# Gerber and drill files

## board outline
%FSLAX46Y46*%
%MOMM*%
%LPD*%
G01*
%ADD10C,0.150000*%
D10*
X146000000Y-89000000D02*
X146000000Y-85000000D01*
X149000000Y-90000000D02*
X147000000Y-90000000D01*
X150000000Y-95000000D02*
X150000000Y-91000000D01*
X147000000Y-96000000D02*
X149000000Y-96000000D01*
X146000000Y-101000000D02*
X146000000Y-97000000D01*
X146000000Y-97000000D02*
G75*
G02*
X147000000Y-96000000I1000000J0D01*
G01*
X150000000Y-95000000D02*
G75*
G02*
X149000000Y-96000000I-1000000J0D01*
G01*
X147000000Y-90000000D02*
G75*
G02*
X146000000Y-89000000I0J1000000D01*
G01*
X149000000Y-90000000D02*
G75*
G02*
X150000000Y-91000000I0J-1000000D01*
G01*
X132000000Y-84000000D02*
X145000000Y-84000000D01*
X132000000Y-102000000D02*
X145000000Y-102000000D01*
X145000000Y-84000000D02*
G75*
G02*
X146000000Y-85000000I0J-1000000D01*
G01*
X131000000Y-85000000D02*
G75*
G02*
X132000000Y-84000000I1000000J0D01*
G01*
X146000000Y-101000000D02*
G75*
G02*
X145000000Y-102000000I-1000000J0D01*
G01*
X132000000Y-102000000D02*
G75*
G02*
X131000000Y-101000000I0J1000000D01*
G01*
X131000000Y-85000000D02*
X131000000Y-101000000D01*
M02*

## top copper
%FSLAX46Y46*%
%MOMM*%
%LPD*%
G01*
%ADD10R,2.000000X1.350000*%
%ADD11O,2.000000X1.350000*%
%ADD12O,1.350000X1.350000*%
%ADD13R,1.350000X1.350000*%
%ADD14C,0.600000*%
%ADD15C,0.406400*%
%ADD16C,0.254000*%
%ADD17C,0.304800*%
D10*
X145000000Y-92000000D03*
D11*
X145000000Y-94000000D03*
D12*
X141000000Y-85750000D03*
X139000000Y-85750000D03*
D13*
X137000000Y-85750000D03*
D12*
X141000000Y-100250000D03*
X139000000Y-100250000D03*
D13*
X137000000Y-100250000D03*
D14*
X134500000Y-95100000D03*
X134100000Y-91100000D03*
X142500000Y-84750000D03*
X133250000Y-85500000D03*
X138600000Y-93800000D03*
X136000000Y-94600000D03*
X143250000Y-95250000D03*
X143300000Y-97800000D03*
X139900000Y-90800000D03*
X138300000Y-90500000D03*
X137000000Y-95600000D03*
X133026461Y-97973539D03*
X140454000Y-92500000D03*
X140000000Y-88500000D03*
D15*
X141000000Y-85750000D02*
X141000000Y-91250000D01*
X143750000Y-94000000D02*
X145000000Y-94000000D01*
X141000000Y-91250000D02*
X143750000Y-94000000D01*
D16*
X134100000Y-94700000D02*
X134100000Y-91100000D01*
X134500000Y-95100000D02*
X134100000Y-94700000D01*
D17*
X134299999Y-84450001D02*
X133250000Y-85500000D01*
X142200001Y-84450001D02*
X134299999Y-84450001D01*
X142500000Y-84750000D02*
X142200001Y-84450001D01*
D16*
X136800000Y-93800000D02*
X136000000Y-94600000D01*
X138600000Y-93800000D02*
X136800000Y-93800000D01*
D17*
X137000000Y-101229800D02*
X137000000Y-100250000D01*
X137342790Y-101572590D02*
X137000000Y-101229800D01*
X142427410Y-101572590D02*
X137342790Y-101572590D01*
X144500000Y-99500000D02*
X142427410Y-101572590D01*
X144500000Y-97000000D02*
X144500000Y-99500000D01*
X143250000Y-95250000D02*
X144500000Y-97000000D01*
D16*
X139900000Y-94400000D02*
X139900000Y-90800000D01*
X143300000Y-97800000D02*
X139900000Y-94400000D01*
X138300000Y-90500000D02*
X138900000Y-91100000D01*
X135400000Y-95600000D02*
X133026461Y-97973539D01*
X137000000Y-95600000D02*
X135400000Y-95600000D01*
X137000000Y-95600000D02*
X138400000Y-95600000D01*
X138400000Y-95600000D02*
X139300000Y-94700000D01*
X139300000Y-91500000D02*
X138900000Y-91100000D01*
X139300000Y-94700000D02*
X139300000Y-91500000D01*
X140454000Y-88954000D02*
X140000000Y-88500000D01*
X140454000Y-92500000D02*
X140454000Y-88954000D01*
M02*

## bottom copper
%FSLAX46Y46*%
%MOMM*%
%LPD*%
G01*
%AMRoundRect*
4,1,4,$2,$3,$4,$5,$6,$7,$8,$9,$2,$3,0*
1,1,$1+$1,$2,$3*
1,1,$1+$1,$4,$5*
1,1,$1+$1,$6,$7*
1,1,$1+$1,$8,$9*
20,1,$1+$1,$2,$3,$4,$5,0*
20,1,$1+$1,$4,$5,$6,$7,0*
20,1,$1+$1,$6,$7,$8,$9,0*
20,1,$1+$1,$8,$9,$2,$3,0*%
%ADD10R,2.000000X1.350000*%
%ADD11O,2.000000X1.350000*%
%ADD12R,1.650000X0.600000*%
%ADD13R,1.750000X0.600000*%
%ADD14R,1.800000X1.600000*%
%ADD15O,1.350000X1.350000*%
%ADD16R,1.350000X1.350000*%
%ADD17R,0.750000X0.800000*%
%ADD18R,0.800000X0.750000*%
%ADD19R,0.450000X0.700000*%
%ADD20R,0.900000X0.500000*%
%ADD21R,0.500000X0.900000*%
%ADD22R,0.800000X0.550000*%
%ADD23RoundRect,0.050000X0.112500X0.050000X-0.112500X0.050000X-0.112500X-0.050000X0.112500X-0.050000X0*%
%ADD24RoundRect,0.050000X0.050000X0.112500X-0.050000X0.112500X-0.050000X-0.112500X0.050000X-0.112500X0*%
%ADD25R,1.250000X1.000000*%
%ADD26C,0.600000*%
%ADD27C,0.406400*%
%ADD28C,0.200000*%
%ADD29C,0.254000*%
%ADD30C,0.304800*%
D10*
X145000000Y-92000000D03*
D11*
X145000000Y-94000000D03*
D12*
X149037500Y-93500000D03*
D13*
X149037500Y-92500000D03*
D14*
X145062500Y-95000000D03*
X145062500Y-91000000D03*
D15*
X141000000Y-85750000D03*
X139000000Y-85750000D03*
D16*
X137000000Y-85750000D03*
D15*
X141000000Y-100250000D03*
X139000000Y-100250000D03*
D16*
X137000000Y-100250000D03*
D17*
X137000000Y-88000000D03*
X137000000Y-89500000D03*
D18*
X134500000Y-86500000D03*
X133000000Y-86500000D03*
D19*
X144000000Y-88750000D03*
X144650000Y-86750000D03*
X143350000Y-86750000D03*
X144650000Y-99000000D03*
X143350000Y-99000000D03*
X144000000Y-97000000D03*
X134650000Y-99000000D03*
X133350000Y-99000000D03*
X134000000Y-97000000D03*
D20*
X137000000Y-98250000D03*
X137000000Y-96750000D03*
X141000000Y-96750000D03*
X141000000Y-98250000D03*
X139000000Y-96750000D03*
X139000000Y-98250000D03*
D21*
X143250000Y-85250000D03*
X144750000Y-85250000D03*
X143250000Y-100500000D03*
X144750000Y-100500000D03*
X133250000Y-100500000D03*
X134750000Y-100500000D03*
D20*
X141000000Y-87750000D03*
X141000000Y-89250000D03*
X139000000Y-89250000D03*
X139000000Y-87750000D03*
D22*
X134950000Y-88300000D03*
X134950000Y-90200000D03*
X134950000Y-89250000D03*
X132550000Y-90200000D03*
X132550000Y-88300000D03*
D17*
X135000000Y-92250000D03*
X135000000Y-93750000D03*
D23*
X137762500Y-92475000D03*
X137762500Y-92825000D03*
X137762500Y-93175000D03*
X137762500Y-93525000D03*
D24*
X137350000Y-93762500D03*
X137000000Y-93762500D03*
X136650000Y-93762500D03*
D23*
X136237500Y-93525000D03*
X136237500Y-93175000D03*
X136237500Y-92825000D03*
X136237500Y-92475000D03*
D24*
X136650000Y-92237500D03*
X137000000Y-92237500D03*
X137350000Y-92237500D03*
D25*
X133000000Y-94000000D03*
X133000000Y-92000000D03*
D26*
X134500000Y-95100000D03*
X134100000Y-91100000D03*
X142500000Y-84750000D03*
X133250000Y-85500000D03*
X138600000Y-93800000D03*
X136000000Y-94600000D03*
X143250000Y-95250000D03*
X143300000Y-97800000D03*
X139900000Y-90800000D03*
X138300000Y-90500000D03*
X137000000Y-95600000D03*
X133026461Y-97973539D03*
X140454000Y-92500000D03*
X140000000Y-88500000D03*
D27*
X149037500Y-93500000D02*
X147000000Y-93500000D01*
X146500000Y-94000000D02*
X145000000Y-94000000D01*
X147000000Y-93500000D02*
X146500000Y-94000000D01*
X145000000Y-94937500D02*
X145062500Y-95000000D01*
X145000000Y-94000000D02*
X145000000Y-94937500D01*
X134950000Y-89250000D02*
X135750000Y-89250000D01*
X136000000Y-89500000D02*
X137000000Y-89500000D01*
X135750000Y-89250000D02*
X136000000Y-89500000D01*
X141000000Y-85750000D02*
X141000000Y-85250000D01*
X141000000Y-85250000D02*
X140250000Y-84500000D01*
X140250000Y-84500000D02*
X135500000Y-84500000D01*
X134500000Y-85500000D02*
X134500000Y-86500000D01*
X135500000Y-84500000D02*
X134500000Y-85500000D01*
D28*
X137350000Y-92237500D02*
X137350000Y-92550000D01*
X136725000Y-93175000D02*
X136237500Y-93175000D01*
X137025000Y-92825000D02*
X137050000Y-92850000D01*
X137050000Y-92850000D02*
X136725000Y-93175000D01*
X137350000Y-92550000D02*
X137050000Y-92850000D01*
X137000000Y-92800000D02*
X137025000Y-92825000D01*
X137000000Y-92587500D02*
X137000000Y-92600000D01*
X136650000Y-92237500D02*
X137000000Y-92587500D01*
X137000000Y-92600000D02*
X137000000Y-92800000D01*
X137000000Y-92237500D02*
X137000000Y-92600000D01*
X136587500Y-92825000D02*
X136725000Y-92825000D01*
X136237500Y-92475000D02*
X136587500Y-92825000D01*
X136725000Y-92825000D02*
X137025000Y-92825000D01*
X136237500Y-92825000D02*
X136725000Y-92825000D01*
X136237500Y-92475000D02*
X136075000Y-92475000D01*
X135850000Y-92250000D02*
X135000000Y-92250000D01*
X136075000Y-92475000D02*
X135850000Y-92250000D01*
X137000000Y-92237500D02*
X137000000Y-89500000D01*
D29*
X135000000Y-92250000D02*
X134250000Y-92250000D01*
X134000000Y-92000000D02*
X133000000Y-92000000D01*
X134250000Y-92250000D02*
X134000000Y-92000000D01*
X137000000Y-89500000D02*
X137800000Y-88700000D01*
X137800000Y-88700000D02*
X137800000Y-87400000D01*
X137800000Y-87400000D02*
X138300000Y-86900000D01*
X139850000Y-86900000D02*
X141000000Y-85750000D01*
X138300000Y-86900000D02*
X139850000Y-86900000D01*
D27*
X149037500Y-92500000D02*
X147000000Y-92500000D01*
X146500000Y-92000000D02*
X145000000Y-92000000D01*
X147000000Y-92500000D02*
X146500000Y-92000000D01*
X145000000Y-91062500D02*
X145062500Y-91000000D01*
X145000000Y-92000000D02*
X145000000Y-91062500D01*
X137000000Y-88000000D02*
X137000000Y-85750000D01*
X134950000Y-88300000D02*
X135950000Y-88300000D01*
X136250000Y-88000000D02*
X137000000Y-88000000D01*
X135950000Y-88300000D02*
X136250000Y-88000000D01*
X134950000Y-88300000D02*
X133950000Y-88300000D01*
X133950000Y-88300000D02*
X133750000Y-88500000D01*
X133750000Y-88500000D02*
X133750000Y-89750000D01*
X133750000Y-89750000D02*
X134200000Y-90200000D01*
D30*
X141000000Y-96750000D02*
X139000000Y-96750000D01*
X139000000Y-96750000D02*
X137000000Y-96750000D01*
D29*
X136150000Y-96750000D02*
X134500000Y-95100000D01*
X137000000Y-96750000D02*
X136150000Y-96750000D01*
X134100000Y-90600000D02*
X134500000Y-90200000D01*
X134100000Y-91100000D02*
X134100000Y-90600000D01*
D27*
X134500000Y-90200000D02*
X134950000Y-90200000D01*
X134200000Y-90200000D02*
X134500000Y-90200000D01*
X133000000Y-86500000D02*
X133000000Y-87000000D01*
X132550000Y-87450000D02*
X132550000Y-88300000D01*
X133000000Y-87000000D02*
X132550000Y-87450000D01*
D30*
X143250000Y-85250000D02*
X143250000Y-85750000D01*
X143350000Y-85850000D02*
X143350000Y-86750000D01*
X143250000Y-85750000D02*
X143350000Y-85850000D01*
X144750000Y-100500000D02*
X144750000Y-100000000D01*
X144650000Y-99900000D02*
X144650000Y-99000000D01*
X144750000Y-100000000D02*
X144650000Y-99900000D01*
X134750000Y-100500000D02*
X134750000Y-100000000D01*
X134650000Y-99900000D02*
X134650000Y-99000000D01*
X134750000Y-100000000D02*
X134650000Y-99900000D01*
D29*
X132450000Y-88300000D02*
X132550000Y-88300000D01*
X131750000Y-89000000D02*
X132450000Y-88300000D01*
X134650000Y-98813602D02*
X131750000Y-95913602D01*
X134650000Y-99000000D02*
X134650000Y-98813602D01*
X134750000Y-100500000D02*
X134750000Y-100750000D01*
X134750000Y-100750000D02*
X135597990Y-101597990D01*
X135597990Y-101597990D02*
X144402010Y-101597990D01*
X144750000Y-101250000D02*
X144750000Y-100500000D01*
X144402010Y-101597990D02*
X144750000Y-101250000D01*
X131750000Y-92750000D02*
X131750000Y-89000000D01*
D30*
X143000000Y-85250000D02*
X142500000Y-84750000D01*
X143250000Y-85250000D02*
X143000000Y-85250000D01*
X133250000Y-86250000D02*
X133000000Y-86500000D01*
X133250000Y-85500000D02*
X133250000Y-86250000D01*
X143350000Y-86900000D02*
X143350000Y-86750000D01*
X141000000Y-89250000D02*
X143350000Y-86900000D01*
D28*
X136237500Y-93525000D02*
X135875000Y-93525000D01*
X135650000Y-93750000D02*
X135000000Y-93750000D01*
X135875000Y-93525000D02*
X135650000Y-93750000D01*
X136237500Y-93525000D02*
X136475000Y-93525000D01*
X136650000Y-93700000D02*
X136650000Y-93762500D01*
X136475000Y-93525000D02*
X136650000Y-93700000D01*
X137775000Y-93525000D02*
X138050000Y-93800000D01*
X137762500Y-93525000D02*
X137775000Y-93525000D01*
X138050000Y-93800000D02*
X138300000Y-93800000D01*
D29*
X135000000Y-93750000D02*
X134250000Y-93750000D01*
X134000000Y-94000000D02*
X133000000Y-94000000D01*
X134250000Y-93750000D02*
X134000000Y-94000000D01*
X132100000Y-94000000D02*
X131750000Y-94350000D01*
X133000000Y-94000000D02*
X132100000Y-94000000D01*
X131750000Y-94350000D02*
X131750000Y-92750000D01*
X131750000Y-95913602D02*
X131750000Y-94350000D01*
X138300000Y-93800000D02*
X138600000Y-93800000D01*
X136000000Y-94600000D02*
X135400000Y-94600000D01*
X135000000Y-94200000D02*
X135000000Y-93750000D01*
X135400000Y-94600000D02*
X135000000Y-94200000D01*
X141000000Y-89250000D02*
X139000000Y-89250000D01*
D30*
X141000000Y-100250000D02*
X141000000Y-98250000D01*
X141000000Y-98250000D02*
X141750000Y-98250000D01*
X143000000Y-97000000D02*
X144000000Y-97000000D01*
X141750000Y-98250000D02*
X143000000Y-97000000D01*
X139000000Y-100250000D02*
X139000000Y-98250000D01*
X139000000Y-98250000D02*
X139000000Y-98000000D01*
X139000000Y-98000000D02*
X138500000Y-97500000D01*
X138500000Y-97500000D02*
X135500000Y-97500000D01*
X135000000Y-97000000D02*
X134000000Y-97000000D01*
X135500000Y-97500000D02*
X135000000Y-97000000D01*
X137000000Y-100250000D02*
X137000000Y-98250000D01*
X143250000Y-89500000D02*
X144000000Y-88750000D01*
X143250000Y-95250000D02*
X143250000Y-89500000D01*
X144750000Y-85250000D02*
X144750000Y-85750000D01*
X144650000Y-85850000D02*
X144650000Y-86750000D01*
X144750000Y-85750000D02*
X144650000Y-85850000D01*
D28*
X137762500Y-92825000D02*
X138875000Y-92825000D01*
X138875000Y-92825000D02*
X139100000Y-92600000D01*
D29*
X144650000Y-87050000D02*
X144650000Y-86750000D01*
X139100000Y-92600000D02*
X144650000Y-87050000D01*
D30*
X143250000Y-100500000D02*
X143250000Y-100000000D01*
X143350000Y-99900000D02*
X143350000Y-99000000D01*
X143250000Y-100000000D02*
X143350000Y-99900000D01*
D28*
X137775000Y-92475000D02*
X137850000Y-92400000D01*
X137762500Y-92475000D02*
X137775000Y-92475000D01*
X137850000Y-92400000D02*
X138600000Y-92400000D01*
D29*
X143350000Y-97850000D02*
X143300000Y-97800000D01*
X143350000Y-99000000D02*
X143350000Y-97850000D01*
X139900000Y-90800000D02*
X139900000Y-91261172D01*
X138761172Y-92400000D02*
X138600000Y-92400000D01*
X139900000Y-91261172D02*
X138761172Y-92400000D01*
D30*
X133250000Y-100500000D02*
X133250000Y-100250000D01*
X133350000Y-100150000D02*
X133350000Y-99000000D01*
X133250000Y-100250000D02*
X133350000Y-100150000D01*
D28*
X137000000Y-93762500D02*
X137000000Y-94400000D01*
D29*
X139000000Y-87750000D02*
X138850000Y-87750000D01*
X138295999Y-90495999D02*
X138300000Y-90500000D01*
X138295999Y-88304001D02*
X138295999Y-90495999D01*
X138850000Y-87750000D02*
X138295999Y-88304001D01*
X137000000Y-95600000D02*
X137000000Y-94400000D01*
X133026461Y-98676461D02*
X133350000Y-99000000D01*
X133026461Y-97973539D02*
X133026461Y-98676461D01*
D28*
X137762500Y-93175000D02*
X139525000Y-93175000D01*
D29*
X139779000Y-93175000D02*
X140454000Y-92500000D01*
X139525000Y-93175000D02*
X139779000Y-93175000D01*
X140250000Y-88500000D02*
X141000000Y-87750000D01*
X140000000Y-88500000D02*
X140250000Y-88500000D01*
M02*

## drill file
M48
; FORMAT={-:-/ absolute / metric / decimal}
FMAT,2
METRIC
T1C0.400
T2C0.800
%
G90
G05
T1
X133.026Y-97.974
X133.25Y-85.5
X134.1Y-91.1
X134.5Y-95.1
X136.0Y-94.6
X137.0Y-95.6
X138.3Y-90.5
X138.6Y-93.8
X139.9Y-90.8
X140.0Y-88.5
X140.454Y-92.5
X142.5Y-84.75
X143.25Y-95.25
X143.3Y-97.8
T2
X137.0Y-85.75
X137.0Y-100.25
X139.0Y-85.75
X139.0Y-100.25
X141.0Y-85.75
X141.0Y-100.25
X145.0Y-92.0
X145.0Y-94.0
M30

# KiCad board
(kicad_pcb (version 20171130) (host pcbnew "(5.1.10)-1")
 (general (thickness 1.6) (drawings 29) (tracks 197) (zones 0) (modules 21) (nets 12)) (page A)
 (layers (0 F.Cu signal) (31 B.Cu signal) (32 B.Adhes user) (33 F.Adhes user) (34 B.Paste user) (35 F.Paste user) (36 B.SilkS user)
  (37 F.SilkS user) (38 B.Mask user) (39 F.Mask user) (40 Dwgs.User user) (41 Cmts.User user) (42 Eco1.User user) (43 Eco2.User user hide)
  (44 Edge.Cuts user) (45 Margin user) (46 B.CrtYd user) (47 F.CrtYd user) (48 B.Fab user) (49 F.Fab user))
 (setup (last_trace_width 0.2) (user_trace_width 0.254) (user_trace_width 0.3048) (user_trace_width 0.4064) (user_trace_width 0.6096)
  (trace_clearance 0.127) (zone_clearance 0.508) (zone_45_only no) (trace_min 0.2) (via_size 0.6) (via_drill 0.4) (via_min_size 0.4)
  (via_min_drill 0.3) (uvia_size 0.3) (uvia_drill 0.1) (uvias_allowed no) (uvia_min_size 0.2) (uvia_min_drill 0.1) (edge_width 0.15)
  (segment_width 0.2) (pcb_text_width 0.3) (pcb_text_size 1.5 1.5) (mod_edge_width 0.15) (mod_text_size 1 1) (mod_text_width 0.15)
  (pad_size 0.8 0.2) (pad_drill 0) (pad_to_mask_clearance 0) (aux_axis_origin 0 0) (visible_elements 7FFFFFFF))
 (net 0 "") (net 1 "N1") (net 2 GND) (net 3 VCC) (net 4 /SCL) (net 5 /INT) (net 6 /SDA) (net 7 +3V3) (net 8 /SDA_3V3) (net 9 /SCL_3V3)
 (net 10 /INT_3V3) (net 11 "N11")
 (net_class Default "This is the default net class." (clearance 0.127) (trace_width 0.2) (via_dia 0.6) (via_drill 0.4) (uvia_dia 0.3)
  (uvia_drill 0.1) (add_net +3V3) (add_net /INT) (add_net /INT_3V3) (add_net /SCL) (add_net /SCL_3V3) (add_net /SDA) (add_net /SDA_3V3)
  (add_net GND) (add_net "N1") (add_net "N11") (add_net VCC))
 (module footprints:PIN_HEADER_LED (layer B.Cu) (at 145 92 180)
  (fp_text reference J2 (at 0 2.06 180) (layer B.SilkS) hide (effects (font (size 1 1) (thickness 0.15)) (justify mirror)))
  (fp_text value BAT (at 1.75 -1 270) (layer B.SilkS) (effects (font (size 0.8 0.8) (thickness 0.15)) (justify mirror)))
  (pad 1 thru_hole rect (at 0 0 180) (size 2 1.35) (drill 0.8) (layers *.Cu *.Mask) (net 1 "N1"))
  (pad 2 thru_hole oval (at 0 -2 180) (size 2 1.35) (drill 0.8) (layers *.Cu *.Mask) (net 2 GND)))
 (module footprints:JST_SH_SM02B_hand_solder (layer B.Cu) (at 147 93 90)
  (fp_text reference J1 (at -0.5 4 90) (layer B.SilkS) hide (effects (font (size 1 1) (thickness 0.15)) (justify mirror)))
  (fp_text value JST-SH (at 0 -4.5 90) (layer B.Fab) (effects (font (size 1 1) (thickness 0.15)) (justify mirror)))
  (pad 1 smd rect (at -0.5 2.0375 90) (size 0.6 1.65) (layers B.Cu B.Paste B.Mask) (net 2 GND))
  (pad 2 smd rect (at 0.5 2.0375 90) (size 0.6 1.75) (layers B.Cu B.Paste B.Mask) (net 1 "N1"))
  (pad 1 smd rect (at -2 -1.9375 90) (size 1.6 1.8) (layers B.Cu B.Paste B.Mask) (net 2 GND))
  (pad 2 smd rect (at 2 -1.9375 90) (size 1.6 1.8) (layers B.Cu B.Paste B.Mask) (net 1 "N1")))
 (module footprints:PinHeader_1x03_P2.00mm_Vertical (layer B.Cu) (at 137 85.75 270)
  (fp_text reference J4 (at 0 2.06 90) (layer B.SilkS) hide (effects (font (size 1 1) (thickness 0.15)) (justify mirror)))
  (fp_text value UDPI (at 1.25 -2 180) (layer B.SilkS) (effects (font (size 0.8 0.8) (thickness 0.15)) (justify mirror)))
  (pad 3 thru_hole oval (at 0 -4 270) (size 1.35 1.35) (drill 0.8) (layers *.Cu *.Mask) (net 2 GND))
  (pad 2 thru_hole oval (at 0 -2 270) (size 1.35 1.35) (drill 0.8) (layers *.Cu *.Mask))
  (pad 1 thru_hole rect (at 0 0 270) (size 1.35 1.35) (drill 0.8) (layers *.Cu *.Mask) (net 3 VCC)))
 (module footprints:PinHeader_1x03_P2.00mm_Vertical (layer B.Cu) (at 137 100.25 270)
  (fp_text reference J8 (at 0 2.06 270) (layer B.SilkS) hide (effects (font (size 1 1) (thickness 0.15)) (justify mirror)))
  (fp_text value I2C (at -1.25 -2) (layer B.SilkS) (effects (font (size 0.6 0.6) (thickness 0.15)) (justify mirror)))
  (pad 3 thru_hole oval (at 0 -4 270) (size 1.35 1.35) (drill 0.8) (layers *.Cu *.Mask) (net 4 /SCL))
  (pad 2 thru_hole oval (at 0 -2 270) (size 1.35 1.35) (drill 0.8) (layers *.Cu *.Mask) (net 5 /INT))
  (pad 1 thru_hole rect (at 0 0 270) (size 1.35 1.35) (drill 0.8) (layers *.Cu *.Mask) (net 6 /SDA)))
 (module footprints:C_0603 (layer B.Cu) (at 137 88.75 270)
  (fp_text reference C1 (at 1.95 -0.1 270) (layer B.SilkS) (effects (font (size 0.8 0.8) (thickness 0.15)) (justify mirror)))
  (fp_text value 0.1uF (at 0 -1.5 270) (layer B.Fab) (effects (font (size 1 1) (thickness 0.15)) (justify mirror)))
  (pad 1 smd rect (at -0.75 0 270) (size 0.8 0.75) (layers B.Cu B.Paste B.Mask) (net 3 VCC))
  (pad 2 smd rect (at 0.75 0 270) (size 0.8 0.75) (layers B.Cu B.Paste B.Mask) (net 2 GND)))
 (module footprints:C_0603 (layer B.Cu) (at 133.75 86.5)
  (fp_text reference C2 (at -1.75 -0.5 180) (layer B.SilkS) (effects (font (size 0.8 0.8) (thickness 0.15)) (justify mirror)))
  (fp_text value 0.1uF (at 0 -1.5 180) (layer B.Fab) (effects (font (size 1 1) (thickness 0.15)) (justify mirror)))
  (pad 2 smd rect (at 0.75 0) (size 0.8 0.75) (layers B.Cu B.Paste B.Mask) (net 2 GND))
  (pad 1 smd rect (at -0.75 0) (size 0.8 0.75) (layers B.Cu B.Paste B.Mask) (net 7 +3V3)))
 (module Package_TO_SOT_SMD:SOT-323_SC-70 (layer B.Cu) (at 144 87.75 270)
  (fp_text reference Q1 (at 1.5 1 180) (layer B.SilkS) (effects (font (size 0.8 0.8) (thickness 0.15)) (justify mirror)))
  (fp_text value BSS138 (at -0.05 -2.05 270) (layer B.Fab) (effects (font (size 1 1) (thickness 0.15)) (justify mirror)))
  (pad 3 smd rect (at 1 0) (size 0.45 0.7) (layers B.Cu B.Paste B.Mask) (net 6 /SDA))
  (pad 2 smd rect (at -1 -0.65) (size 0.45 0.7) (layers B.Cu B.Paste B.Mask) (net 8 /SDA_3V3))
  (pad 1 smd rect (at -1 0.65) (size 0.45 0.7) (layers B.Cu B.Paste B.Mask) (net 7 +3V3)))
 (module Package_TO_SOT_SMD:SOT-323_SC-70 (layer B.Cu) (at 144 98 90)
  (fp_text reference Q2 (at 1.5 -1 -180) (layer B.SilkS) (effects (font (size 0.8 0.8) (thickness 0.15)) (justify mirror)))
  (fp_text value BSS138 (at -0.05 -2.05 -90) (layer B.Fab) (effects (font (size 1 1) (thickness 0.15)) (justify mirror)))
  (pad 1 smd rect (at -1 0.65 180) (size 0.45 0.7) (layers B.Cu B.Paste B.Mask) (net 7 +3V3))
  (pad 2 smd rect (at -1 -0.65 180) (size 0.45 0.7) (layers B.Cu B.Paste B.Mask) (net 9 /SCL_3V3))
  (pad 3 smd rect (at 1 0 180) (size 0.45 0.7) (layers B.Cu B.Paste B.Mask) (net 4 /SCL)))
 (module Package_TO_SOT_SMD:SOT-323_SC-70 (layer B.Cu) (at 134 98 90)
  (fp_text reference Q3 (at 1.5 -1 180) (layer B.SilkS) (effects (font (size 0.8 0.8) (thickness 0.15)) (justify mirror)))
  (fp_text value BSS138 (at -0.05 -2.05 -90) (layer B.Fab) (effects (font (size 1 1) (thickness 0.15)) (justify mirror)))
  (pad 1 smd rect (at -1 0.65 180) (size 0.45 0.7) (layers B.Cu B.Paste B.Mask) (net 7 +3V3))
  (pad 2 smd rect (at -1 -0.65 180) (size 0.45 0.7) (layers B.Cu B.Paste B.Mask) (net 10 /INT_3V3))
  (pad 3 smd rect (at 1 0 180) (size 0.45 0.7) (layers B.Cu B.Paste B.Mask) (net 5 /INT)))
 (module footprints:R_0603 (layer B.Cu) (at 137 97.5 270)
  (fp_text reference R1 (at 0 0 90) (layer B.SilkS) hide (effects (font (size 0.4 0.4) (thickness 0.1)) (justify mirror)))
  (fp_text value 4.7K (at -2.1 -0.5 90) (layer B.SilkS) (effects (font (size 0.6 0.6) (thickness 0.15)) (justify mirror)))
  (pad 2 smd rect (at 0.75 0 270) (size 0.5 0.9) (layers B.Cu B.Paste B.Mask) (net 6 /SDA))
  (pad 1 smd rect (at -0.75 0 270) (size 0.5 0.9) (layers B.Cu B.Paste B.Mask) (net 3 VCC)))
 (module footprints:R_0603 (layer B.Cu) (at 141 97.5 270)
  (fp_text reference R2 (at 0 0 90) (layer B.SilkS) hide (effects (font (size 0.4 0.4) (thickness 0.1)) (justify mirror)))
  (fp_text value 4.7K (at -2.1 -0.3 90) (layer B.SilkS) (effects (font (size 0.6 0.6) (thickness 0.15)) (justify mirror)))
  (pad 1 smd rect (at -0.75 0 270) (size 0.5 0.9) (layers B.Cu B.Paste B.Mask) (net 3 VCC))
  (pad 2 smd rect (at 0.75 0 270) (size 0.5 0.9) (layers B.Cu B.Paste B.Mask) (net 4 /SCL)))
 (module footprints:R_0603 (layer B.Cu) (at 139 97.5 270)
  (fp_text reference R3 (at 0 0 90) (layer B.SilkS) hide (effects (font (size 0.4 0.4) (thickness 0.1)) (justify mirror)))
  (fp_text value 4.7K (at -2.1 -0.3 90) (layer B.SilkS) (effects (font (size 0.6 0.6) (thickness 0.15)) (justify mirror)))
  (pad 1 smd rect (at -0.75 0 270) (size 0.5 0.9) (layers B.Cu B.Paste B.Mask) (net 3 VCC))
  (pad 2 smd rect (at 0.75 0 270) (size 0.5 0.9) (layers B.Cu B.Paste B.Mask) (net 5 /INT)))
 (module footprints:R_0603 (layer B.Cu) (at 144 85.25)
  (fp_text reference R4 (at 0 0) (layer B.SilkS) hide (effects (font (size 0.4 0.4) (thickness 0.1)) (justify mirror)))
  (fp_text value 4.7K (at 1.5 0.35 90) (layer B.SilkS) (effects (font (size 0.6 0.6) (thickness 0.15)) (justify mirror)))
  (pad 1 smd rect (at -0.75 0) (size 0.5 0.9) (layers B.Cu B.Paste B.Mask) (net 7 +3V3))
  (pad 2 smd rect (at 0.75 0) (size 0.5 0.9) (layers B.Cu B.Paste B.Mask) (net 8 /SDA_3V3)))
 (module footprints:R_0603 (layer B.Cu) (at 144 100.5 180)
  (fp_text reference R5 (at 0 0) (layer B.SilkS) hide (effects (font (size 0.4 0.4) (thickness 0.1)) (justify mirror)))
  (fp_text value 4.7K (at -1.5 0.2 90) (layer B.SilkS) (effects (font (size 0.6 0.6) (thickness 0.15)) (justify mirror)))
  (pad 2 smd rect (at 0.75 0 180) (size 0.5 0.9) (layers B.Cu B.Paste B.Mask) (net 9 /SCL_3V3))
  (pad 1 smd rect (at -0.75 0 180) (size 0.5 0.9) (layers B.Cu B.Paste B.Mask) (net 7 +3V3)))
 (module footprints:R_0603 (layer B.Cu) (at 134 100.5 180)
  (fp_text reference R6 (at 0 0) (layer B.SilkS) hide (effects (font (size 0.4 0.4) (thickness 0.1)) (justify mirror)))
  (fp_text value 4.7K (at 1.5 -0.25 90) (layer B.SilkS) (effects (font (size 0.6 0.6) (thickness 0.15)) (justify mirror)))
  (pad 2 smd rect (at 0.75 0 180) (size 0.5 0.9) (layers B.Cu B.Paste B.Mask) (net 10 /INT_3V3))
  (pad 1 smd rect (at -0.75 0 180) (size 0.5 0.9) (layers B.Cu B.Paste B.Mask) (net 7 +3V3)))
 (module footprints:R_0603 (layer B.Cu) (at 141 88.5 90)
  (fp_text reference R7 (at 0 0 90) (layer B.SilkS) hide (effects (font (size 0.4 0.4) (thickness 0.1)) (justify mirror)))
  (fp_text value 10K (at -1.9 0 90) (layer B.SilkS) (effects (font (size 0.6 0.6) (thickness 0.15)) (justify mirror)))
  (pad 2 smd rect (at 0.75 0 90) (size 0.5 0.9) (layers B.Cu B.Paste B.Mask) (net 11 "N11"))
  (pad 1 smd rect (at -0.75 0 90) (size 0.5 0.9) (layers B.Cu B.Paste B.Mask) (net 7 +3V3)))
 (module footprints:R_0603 (layer B.Cu) (at 139 88.5 90)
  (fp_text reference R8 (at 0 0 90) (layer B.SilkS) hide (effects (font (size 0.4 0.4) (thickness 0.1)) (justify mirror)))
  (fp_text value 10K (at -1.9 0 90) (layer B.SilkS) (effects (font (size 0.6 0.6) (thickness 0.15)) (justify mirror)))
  (pad 1 smd rect (at -0.75 0 90) (size 0.5 0.9) (layers B.Cu B.Paste B.Mask) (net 7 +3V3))
  (pad 2 smd rect (at 0.75 0 90) (size 0.5 0.9) (layers B.Cu B.Paste B.Mask) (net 10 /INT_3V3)))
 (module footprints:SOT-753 (layer B.Cu) (at 133.75 89.25 270) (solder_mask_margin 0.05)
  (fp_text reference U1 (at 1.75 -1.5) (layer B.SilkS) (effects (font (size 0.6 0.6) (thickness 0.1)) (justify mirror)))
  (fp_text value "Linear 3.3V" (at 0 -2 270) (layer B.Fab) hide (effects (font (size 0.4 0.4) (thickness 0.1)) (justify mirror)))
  (pad 1 smd rect (at -0.95 -1.2 270) (size 0.55 0.8) (layers B.Cu B.Paste B.Mask) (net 3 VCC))
  (pad 3 smd rect (at 0.95 -1.2 270) (size 0.55 0.8) (layers B.Cu B.Paste B.Mask) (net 3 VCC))
  (pad 2 smd rect (at 0 -1.2 270) (size 0.55 0.8) (layers B.Cu B.Paste B.Mask) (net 2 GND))
  (pad 4 smd rect (at 0.95 1.2 270) (size 0.55 0.8) (layers B.Cu B.Paste B.Mask))
  (pad 5 smd rect (at -0.95 1.2 270) (size 0.55 0.8) (layers B.Cu B.Paste B.Mask) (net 7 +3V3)))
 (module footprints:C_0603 (layer B.Cu) (at 135 93 90)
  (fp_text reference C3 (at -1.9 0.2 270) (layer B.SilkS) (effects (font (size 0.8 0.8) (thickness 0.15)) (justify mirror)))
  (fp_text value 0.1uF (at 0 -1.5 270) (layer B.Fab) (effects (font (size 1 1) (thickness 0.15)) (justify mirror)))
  (pad 2 smd rect (at 0.75 0 90) (size 0.8 0.75) (layers B.Cu B.Paste B.Mask) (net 2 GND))
  (pad 1 smd rect (at -0.75 0 90) (size 0.8 0.75) (layers B.Cu B.Paste B.Mask) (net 7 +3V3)))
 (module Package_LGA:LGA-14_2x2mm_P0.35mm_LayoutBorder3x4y (layer B.Cu) (at 137 93 180) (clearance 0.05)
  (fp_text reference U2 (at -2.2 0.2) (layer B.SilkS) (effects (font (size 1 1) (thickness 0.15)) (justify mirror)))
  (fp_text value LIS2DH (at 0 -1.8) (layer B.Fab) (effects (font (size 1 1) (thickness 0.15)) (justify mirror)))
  (pad 1 smd roundrect (at -0.7625 0.525 180) (size 0.325 0.2) (layers B.Cu B.Paste B.Mask) (roundrect_rratio 0.25) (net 9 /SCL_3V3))
  (pad 2 smd roundrect (at -0.7625 0.175 180) (size 0.325 0.2) (layers B.Cu B.Paste B.Mask) (roundrect_rratio 0.25) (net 8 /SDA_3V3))
  (pad 3 smd roundrect (at -0.7625 -0.175 180) (size 0.325 0.2) (layers B.Cu B.Paste B.Mask) (roundrect_rratio 0.25) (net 11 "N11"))
  (pad 4 smd roundrect (at -0.7625 -0.525 180) (size 0.325 0.2) (layers B.Cu B.Paste B.Mask) (roundrect_rratio 0.25) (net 7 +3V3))
  (pad 5 smd roundrect (at -0.35 -0.7625 180) (size 0.2 0.325) (layers B.Cu B.Paste B.Mask) (roundrect_rratio 0.25))
  (pad 6 smd roundrect (at 0 -0.7625 180) (size 0.2 0.325) (layers B.Cu B.Paste B.Mask) (roundrect_rratio 0.25) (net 10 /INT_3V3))
  (pad 7 smd roundrect (at 0.35 -0.7625 180) (size 0.2 0.325) (layers B.Cu B.Paste B.Mask) (roundrect_rratio 0.25) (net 7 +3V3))
  (pad 8 smd roundrect (at 0.7625 -0.525 180) (size 0.325 0.2) (layers B.Cu B.Paste B.Mask) (roundrect_rratio 0.25) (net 7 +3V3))
  (pad 9 smd roundrect (at 0.7625 -0.175 180) (size 0.325 0.2) (layers B.Cu B.Paste B.Mask) (roundrect_rratio 0.25) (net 2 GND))
  (pad 10 smd roundrect (at 0.7625 0.175 180) (size 0.325 0.2) (layers B.Cu B.Paste B.Mask) (roundrect_rratio 0.25) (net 2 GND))
  (pad 11 smd roundrect (at 0.7625 0.525 180) (size 0.325 0.2) (layers B.Cu B.Paste B.Mask) (roundrect_rratio 0.25) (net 2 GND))
  (pad 12 smd roundrect (at 0.35 0.7625 180) (size 0.2 0.325) (layers B.Cu B.Paste B.Mask) (roundrect_rratio 0.25) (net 2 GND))
  (pad 13 smd roundrect (at 0 0.7625 180) (size 0.2 0.325) (layers B.Cu B.Paste B.Mask) (roundrect_rratio 0.25) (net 2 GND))
  (pad 14 smd roundrect (at -0.35 0.7625 180) (size 0.2 0.325) (layers B.Cu B.Paste B.Mask) (roundrect_rratio 0.25) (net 2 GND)))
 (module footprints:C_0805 (layer B.Cu) (at 133 93 90)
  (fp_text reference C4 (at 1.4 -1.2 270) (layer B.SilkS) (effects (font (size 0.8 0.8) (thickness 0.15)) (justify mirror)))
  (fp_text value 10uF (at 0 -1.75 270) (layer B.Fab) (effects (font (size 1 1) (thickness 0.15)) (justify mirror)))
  (pad 1 smd rect (at -1 0 90) (size 1 1.25) (layers B.Cu B.Paste B.Mask) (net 7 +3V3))
  (pad 2 smd rect (at 1 0 90) (size 1 1.25) (layers B.Cu B.Paste B.Mask) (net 2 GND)))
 (gr_line (start 146 89) (end 146 85) (layer Edge.Cuts) (width 0.15))
 (gr_line (start 149 90) (end 147 90) (layer Edge.Cuts) (width 0.15))
 (gr_line (start 150 95) (end 150 91) (layer Edge.Cuts) (width 0.15))
 (gr_line (start 147 96) (end 149 96) (layer Edge.Cuts) (width 0.15))
 (gr_line (start 146 101) (end 146 97) (layer Edge.Cuts) (width 0.15))
 (gr_arc (start 147 97) (end 147 96) (angle -90) (layer Edge.Cuts) (width 0.15))
 (gr_arc (start 149 95) (end 149 96) (angle -90) (layer Edge.Cuts) (width 0.15))
 (gr_arc (start 147 89) (end 146 89) (angle -90) (layer Edge.Cuts) (width 0.15))
 (gr_arc (start 149 91) (end 150 91) (angle -90) (layer Edge.Cuts) (width 0.15))
 (gr_line (start 132 84) (end 145 84) (layer Edge.Cuts) (width 0.15))
 (gr_line (start 132 102) (end 145 102) (layer Edge.Cuts) (width 0.15))
 (gr_arc (start 145 85) (end 145 84) (angle 90) (layer Edge.Cuts) (width 0.15))
 (gr_arc (start 132 85) (end 131 85) (angle 90) (layer Edge.Cuts) (width 0.15))
 (gr_arc (start 145 101) (end 146 101) (angle 90) (layer Edge.Cuts) (width 0.15))
 (gr_arc (start 132 101) (end 132 102) (angle 90) (layer Edge.Cuts) (width 0.15))
 (gr_line (start 131 85) (end 131 101) (angle 90) (layer Edge.Cuts) (width 0.15))
 (segment (start 149.0375 93.5) (end 147 93.5) (width 0.4064) (layer B.Cu) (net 2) (status 10))
 (segment (start 146.5 94) (end 145 94) (width 0.4064) (layer B.Cu) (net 2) (status 20))
 (segment (start 147 93.5) (end 146.5 94) (width 0.4064) (layer B.Cu) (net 2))
 (segment (start 145 94.9375) (end 145.0625 95) (width 0.4064) (layer B.Cu) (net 2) (status 30))
 (segment (start 145 94) (end 145 94.9375) (width 0.4064) (layer B.Cu) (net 2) (status 30))
 (segment (start 134.95 89.25) (end 135.75 89.25) (width 0.4064) (layer B.Cu) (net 2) (status 10))
 (segment (start 136 89.5) (end 137 89.5) (width 0.4064) (layer B.Cu) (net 2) (status 20))
 (segment (start 135.75 89.25) (end 136 89.5) (width 0.4064) (layer B.Cu) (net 2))
 (segment (start 141 85.75) (end 141 85.25) (width 0.4064) (layer B.Cu) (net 2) (status 30))
 (segment (start 141 85.25) (end 140.25 84.5) (width 0.4064) (layer B.Cu) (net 2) (status 10))
 (segment (start 140.25 84.5) (end 135.5 84.5) (width 0.4064) (layer B.Cu) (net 2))
 (segment (start 134.5 85.5) (end 134.5 86.5) (width 0.4064) (layer B.Cu) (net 2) (status 20))
 (segment (start 135.5 84.5) (end 134.5 85.5) (width 0.4064) (layer B.Cu) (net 2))
 (segment (start 141 85.75) (end 141 91.25) (width 0.4064) (layer F.Cu) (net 2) (status 10))
 (segment (start 143.75 94) (end 145 94) (width 0.4064) (layer F.Cu) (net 2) (status 20))
 (segment (start 141 91.25) (end 143.75 94) (width 0.4064) (layer F.Cu) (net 2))
 (segment (start 137.35 92.2375) (end 137.35 92.55) (width 0.2) (layer B.Cu) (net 2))
 (segment (start 136.725 93.175) (end 136.2375 93.175) (width 0.2) (layer B.Cu) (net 2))
 (segment (start 137.025 92.825) (end 137.05 92.85) (width 0.2) (layer B.Cu) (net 2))
 (segment (start 137.05 92.85) (end 136.725 93.175) (width 0.2) (layer B.Cu) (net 2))
 (segment (start 137.35 92.55) (end 137.05 92.85) (width 0.2) (layer B.Cu) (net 2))
 (segment (start 137 92.8) (end 137.025 92.825) (width 0.2) (layer B.Cu) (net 2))
 (segment (start 137 92.5875) (end 137 92.6) (width 0.2) (layer B.Cu) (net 2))
 (segment (start 136.65 92.2375) (end 137 92.5875) (width 0.2) (layer B.Cu) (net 2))
 (segment (start 137 92.6) (end 137 92.8) (width 0.2) (layer B.Cu) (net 2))
 (segment (start 137 92.2375) (end 137 92.6) (width 0.2) (layer B.Cu) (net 2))
 (segment (start 136.5875 92.825) (end 136.725 92.825) (width 0.2) (layer B.Cu) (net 2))
 (segment (start 136.2375 92.475) (end 136.5875 92.825) (width 0.2) (layer B.Cu) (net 2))
 (segment (start 136.725 92.825) (end 137.025 92.825) (width 0.2) (layer B.Cu) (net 2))
 (segment (start 136.2375 92.825) (end 136.725 92.825) (width 0.2) (layer B.Cu) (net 2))
 (segment (start 136.2375 92.475) (end 136.075 92.475) (width 0.2) (layer B.Cu) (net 2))
 (segment (start 135.85 92.25) (end 135 92.25) (width 0.2) (layer B.Cu) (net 2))
 (segment (start 136.075 92.475) (end 135.85 92.25) (width 0.2) (layer B.Cu) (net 2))
 (segment (start 137 92.2375) (end 137 89.5) (width 0.2) (layer B.Cu) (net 2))
 (segment (start 135 92.25) (end 134.25 92.25) (width 0.254) (layer B.Cu) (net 2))
 (segment (start 134 92) (end 133 92) (width 0.254) (layer B.Cu) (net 2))
 (segment (start 134.25 92.25) (end 134 92) (width 0.254) (layer B.Cu) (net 2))
 (segment (start 137 89.5) (end 137.8 88.7) (width 0.254) (layer B.Cu) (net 2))
 (segment (start 137.8 88.7) (end 137.8 87.4) (width 0.254) (layer B.Cu) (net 2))
 (segment (start 137.8 87.4) (end 138.3 86.9) (width 0.254) (layer B.Cu) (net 2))
 (segment (start 139.85 86.9) (end 141 85.75) (width 0.254) (layer B.Cu) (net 2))
 (segment (start 138.3 86.9) (end 139.85 86.9) (width 0.254) (layer B.Cu) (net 2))
 (segment (start 149.0375 92.5) (end 147 92.5) (width 0.4064) (layer B.Cu) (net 1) (status 10))
 (segment (start 146.5 92) (end 145 92) (width 0.4064) (layer B.Cu) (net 1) (status 20))
 (segment (start 147 92.5) (end 146.5 92) (width 0.4064) (layer B.Cu) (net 1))
 (segment (start 145 91.0625) (end 145.0625 91) (width 0.4064) (layer B.Cu) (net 1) (status 30))
 (segment (start 145 92) (end 145 91.0625) (width 0.4064) (layer B.Cu) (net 1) (status 30))
 (segment (start 137 88) (end 137 85.75) (width 0.4064) (layer B.Cu) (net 3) (status 30))
 (segment (start 134.95 88.3) (end 135.95 88.3) (width 0.4064) (layer B.Cu) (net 3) (status 10))
 (segment (start 136.25 88) (end 137 88) (width 0.4064) (layer B.Cu) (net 3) (status 20))
 (segment (start 135.95 88.3) (end 136.25 88) (width 0.4064) (layer B.Cu) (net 3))
 (segment (start 134.95 88.3) (end 133.95 88.3) (width 0.4064) (layer B.Cu) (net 3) (status 10))
 (segment (start 133.95 88.3) (end 133.75 88.5) (width 0.4064) (layer B.Cu) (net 3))
 (segment (start 133.75 88.5) (end 133.75 89.75) (width 0.4064) (layer B.Cu) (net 3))
 (segment (start 133.75 89.75) (end 134.2 90.2) (width 0.4064) (layer B.Cu) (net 3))
 (segment (start 141 96.75) (end 139 96.75) (width 0.3048) (layer B.Cu) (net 3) (status 30))
 (segment (start 139 96.75) (end 137 96.75) (width 0.3048) (layer B.Cu) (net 3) (status 30))
 (via (at 134.5 95.1) (size 0.6) (drill 0.4) (layers F.Cu B.Cu) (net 3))
 (segment (start 136.15 96.75) (end 134.5 95.1) (width 0.254) (layer B.Cu) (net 3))
 (segment (start 137 96.75) (end 136.15 96.75) (width 0.254) (layer B.Cu) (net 3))
 (via (at 134.1 91.1) (size 0.6) (drill 0.4) (layers F.Cu B.Cu) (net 3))
 (segment (start 134.1 94.7) (end 134.1 91.1) (width 0.254) (layer F.Cu) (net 3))
 (segment (start 134.5 95.1) (end 134.1 94.7) (width 0.254) (layer F.Cu) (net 3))
 (segment (start 134.1 90.6) (end 134.5 90.2) (width 0.254) (layer B.Cu) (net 3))
 (segment (start 134.1 91.1) (end 134.1 90.6) (width 0.254) (layer B.Cu) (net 3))
 (segment (start 134.5 90.2) (end 134.95 90.2) (width 0.4064) (layer B.Cu) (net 3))
 (segment (start 134.2 90.2) (end 134.5 90.2) (width 0.4064) (layer B.Cu) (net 3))
 (segment (start 133 86.5) (end 133 87) (width 0.4064) (layer B.Cu) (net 7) (status 10))
 (segment (start 132.55 87.45) (end 132.55 88.3) (width 0.4064) (layer B.Cu) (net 7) (status 20))
 (segment (start 133 87) (end 132.55 87.45) (width 0.4064) (layer B.Cu) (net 7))
 (segment (start 143.25 85.25) (end 143.25 85.75) (width 0.3048) (layer B.Cu) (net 7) (status 10))
 (segment (start 143.35 85.85) (end 143.35 86.75) (width 0.3048) (layer B.Cu) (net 7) (status 20))
 (segment (start 143.25 85.75) (end 143.35 85.85) (width 0.3048) (layer B.Cu) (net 7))
 (segment (start 144.75 100.5) (end 144.75 100) (width 0.3048) (layer B.Cu) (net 7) (status 10))
 (segment (start 144.65 99.9) (end 144.65 99) (width 0.3048) (layer B.Cu) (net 7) (status 20))
 (segment (start 144.75 100) (end 144.65 99.9) (width 0.3048) (layer B.Cu) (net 7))
 (segment (start 134.75 100.5) (end 134.75 100) (width 0.3048) (layer B.Cu) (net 7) (status 10))
 (segment (start 134.65 99.9) (end 134.65 99) (width 0.3048) (layer B.Cu) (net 7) (status 20))
 (segment (start 134.75 100) (end 134.65 99.9) (width 0.3048) (layer B.Cu) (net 7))
 (segment (start 132.45 88.3) (end 132.55 88.3) (width 0.254) (layer B.Cu) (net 7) (status 30))
 (segment (start 131.75 89) (end 132.45 88.3) (width 0.254) (layer B.Cu) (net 7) (status 20))
 (segment (start 134.65 98.813602) (end 131.75 95.913602) (width 0.254) (layer B.Cu) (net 7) (status 10))
 (segment (start 134.65 99) (end 134.65 98.813602) (width 0.254) (layer B.Cu) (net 7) (status 30))
 (segment (start 134.75 100.5) (end 134.75 100.75) (width 0.254) (layer B.Cu) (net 7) (status 30))
 (segment (start 134.75 100.75) (end 135.59799 101.59799) (width 0.254) (layer B.Cu) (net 7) (status 10))
 (segment (start 135.59799 101.59799) (end 144.40201 101.59799) (width 0.254) (layer B.Cu) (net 7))
 (segment (start 144.75 101.25) (end 144.75 100.5) (width 0.254) (layer B.Cu) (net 7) (status 20))
 (segment (start 144.40201 101.59799) (end 144.75 101.25) (width 0.254) (layer B.Cu) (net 7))
 (segment (start 131.75 92.75) (end 131.75 89) (width 0.254) (layer B.Cu) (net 7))
 (via (at 142.5 84.75) (size 0.6) (drill 0.4) (layers F.Cu B.Cu) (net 7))
 (segment (start 143 85.25) (end 142.5 84.75) (width 0.3048) (layer B.Cu) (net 7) (status 10))
 (segment (start 143.25 85.25) (end 143 85.25) (width 0.3048) (layer B.Cu) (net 7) (status 30))
 (via (at 133.25 85.5) (size 0.6) (drill 0.4) (layers F.Cu B.Cu) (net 7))
 (segment (start 134.299999 84.450001) (end 133.25 85.5) (width 0.3048) (layer F.Cu) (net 7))
 (segment (start 142.200001 84.450001) (end 134.299999 84.450001) (width 0.3048) (layer F.Cu) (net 7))
 (segment (start 142.5 84.75) (end 142.200001 84.450001) (width 0.3048) (layer F.Cu) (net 7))
 (segment (start 133.25 86.25) (end 133 86.5) (width 0.3048) (layer B.Cu) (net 7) (status 30))
 (segment (start 133.25 85.5) (end 133.25 86.25) (width 0.3048) (layer B.Cu) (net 7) (status 20))
 (segment (start 143.35 86.9) (end 143.35 86.75) (width 0.3048) (layer B.Cu) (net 7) (status 30))
 (segment (start 141 89.25) (end 143.35 86.9) (width 0.3048) (layer B.Cu) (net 7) (status 30))
 (segment (start 136.2375 93.525) (end 135.875 93.525) (width 0.2) (layer B.Cu) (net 7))
 (segment (start 135.65 93.75) (end 135 93.75) (width 0.2) (layer B.Cu) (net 7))
 (segment (start 135.875 93.525) (end 135.65 93.75) (width 0.2) (layer B.Cu) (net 7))
 (segment (start 136.2375 93.525) (end 136.475 93.525) (width 0.2) (layer B.Cu) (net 7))
 (segment (start 136.65 93.7) (end 136.65 93.7625) (width 0.2) (layer B.Cu) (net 7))
 (segment (start 136.475 93.525) (end 136.65 93.7) (width 0.2) (layer B.Cu) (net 7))
 (segment (start 137.775 93.525) (end 138.05 93.8) (width 0.2) (layer B.Cu) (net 7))
 (segment (start 137.7625 93.525) (end 137.775 93.525) (width 0.2) (layer B.Cu) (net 7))
 (segment (start 138.05 93.8) (end 138.3 93.8) (width 0.2) (layer B.Cu) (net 7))
 (segment (start 135 93.75) (end 134.25 93.75) (width 0.254) (layer B.Cu) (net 7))
 (segment (start 134 94) (end 133 94) (width 0.254) (layer B.Cu) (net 7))
 (segment (start 134.25 93.75) (end 134 94) (width 0.254) (layer B.Cu) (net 7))
 (segment (start 132.1 94) (end 131.75 94.35) (width 0.254) (layer B.Cu) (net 7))
 (segment (start 133 94) (end 132.1 94) (width 0.254) (layer B.Cu) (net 7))
 (segment (start 131.75 94.35) (end 131.75 92.75) (width 0.254) (layer B.Cu) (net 7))
 (segment (start 131.75 95.913602) (end 131.75 94.35) (width 0.254) (layer B.Cu) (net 7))
 (via (at 138.6 93.8) (size 0.6) (drill 0.4) (layers F.Cu B.Cu) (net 7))
 (segment (start 138.3 93.8) (end 138.6 93.8) (width 0.254) (layer B.Cu) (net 7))
 (via (at 136 94.6) (size 0.6) (drill 0.4) (layers F.Cu B.Cu) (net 7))
 (segment (start 136.8 93.8) (end 136 94.6) (width 0.254) (layer F.Cu) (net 7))
 (segment (start 138.6 93.8) (end 136.8 93.8) (width 0.254) (layer F.Cu) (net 7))
 (segment (start 136 94.6) (end 135.4 94.6) (width 0.254) (layer B.Cu) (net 7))
 (segment (start 135 94.2) (end 135 93.75) (width 0.254) (layer B.Cu) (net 7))
 (segment (start 135.4 94.6) (end 135 94.2) (width 0.254) (layer B.Cu) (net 7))
 (segment (start 141 89.25) (end 139 89.25) (width 0.254) (layer B.Cu) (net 7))
 (segment (start 141 100.25) (end 141 98.25) (width 0.3048) (layer B.Cu) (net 4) (status 30))
 (segment (start 141 98.25) (end 141.75 98.25) (width 0.3048) (layer B.Cu) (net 4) (status 10))
 (segment (start 143 97) (end 144 97) (width 0.3048) (layer B.Cu) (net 4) (status 20))
 (segment (start 141.75 98.25) (end 143 97) (width 0.3048) (layer B.Cu) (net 4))
 (segment (start 139 100.25) (end 139 98.25) (width 0.3048) (layer B.Cu) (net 5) (status 30))
 (segment (start 139 98.25) (end 139 98) (width 0.3048) (layer B.Cu) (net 5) (status 30))
 (segment (start 139 98) (end 138.5 97.5) (width 0.3048) (layer B.Cu) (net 5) (status 10))
 (segment (start 138.5 97.5) (end 135.5 97.5) (width 0.3048) (layer B.Cu) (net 5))
 (segment (start 135 97) (end 134 97) (width 0.3048) (layer B.Cu) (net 5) (status 20))
 (segment (start 135.5 97.5) (end 135 97) (width 0.3048) (layer B.Cu) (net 5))
 (segment (start 137 100.25) (end 137 98.25) (width 0.3048) (layer B.Cu) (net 6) (status 30))
 (segment (start 143.25 89.5) (end 144 88.75) (width 0.3048) (layer B.Cu) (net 6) (status 20))
 (segment (start 143.25 95.25) (end 143.25 89.5) (width 0.3048) (layer B.Cu) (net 6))
 (segment (start 137 101.2298) (end 137 100.25) (width 0.3048) (layer F.Cu) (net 6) (status 20))
 (segment (start 137.34279 101.57259) (end 137 101.2298) (width 0.3048) (layer F.Cu) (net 6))
 (segment (start 142.42741 101.57259) (end 137.34279 101.57259) (width 0.3048) (layer F.Cu) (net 6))
 (segment (start 144.5 99.5) (end 142.42741 101.57259) (width 0.3048) (layer F.Cu) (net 6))
 (segment (start 144.5 97) (end 144.5 99.5) (width 0.3048) (layer F.Cu) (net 6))
 (segment (start 143.25 95.25) (end 144.5 97) (width 0.3048) (layer F.Cu) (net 6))
 (via (at 143.25 95.25) (size 0.6) (drill 0.4) (layers F.Cu B.Cu) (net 6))
 (segment (start 144.75 85.25) (end 144.75 85.75) (width 0.3048) (layer B.Cu) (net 8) (status 10))
 (segment (start 144.65 85.85) (end 144.65 86.75) (width 0.3048) (layer B.Cu) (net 8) (status 20))
 (segment (start 144.75 85.75) (end 144.65 85.85) (width 0.3048) (layer B.Cu) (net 8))
 (segment (start 137.7625 92.825) (end 138.875 92.825) (width 0.2) (layer B.Cu) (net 8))
 (segment (start 138.875 92.825) (end 139.1 92.6) (width 0.2) (layer B.Cu) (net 8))
 (segment (start 144.65 87.05) (end 144.65 86.75) (width 0.254) (layer B.Cu) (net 8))
 (segment (start 139.1 92.6) (end 144.65 87.05) (width 0.254) (layer B.Cu) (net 8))
 (segment (start 143.25 100.5) (end 143.25 100) (width 0.3048) (layer B.Cu) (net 9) (status 10))
 (segment (start 143.35 99.9) (end 143.35 99) (width 0.3048) (layer B.Cu) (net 9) (status 20))
 (segment (start 143.25 100) (end 143.35 99.9) (width 0.3048) (layer B.Cu) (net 9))
 (segment (start 137.775 92.475) (end 137.85 92.4) (width 0.2) (layer B.Cu) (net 9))
 (segment (start 137.7625 92.475) (end 137.775 92.475) (width 0.2) (layer B.Cu) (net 9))
 (segment (start 137.85 92.4) (end 138.6 92.4) (width 0.2) (layer B.Cu) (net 9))
 (via (at 143.3 97.8) (size 0.6) (drill 0.4) (layers F.Cu B.Cu) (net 9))
 (segment (start 143.35 97.85) (end 143.3 97.8) (width 0.254) (layer B.Cu) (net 9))
 (segment (start 143.35 99) (end 143.35 97.85) (width 0.254) (layer B.Cu) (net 9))
 (segment (start 139.9 94.4) (end 139.9 90.8) (width 0.254) (layer F.Cu) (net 9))
 (via (at 139.9 90.8) (size 0.6) (drill 0.4) (layers F.Cu B.Cu) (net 9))
 (segment (start 143.3 97.8) (end 139.9 94.4) (width 0.254) (layer F.Cu) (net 9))
 (segment (start 139.9 90.8) (end 139.9 91.261172) (width 0.254) (layer B.Cu) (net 9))
 (segment (start 138.761172 92.4) (end 138.6 92.4) (width 0.254) (layer B.Cu) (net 9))
 (segment (start 139.9 91.261172) (end 138.761172 92.4) (width 0.254) (layer B.Cu) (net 9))
 (segment (start 133.25 100.5) (end 133.25 100.25) (width 0.3048) (layer B.Cu) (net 10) (status 30))
 (segment (start 133.35 100.15) (end 133.35 99) (width 0.3048) (layer B.Cu) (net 10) (status 30))
 (segment (start 133.25 100.25) (end 133.35 100.15) (width 0.3048) (layer B.Cu) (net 10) (status 30))
 (segment (start 137 93.7625) (end 137 94.4) (width 0.2) (layer B.Cu) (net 10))
 (segment (start 139 87.75) (end 138.85 87.75) (width 0.254) (layer B.Cu) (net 10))
 (via (at 138.3 90.5) (size 0.6) (drill 0.4) (layers F.Cu B.Cu) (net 10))
 (segment (start 138.295999 90.495999) (end 138.3 90.5) (width 0.254) (layer B.Cu) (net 10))
 (segment (start 138.295999 88.304001) (end 138.295999 90.495999) (width 0.254) (layer B.Cu) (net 10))
 (segment (start 138.85 87.75) (end 138.295999 88.304001) (width 0.254) (layer B.Cu) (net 10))
 (segment (start 138.3 90.5) (end 138.9 91.1) (width 0.254) (layer F.Cu) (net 10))
 (via (at 137 95.6) (size 0.6) (drill 0.4) (layers F.Cu B.Cu) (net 10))
 (segment (start 137 95.6) (end 137 94.4) (width 0.254) (layer B.Cu) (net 10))
 (via (at 133.026461 97.973539) (size 0.6) (drill 0.4) (layers F.Cu B.Cu) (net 10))
 (segment (start 135.4 95.6) (end 133.026461 97.973539) (width 0.254) (layer F.Cu) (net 10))
 (segment (start 137 95.6) (end 135.4 95.6) (width 0.254) (layer F.Cu) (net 10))
 (segment (start 133.026461 98.676461) (end 133.35 99) (width 0.254) (layer B.Cu) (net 10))
 (segment (start 133.026461 97.973539) (end 133.026461 98.676461) (width 0.254) (layer B.Cu) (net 10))
 (segment (start 137 95.6) (end 138.4 95.6) (width 0.254) (layer F.Cu) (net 10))
 (segment (start 138.4 95.6) (end 139.3 94.7) (width 0.254) (layer F.Cu) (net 10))
 (segment (start 139.3 91.5) (end 138.9 91.1) (width 0.254) (layer F.Cu) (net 10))
 (segment (start 139.3 94.7) (end 139.3 91.5) (width 0.254) (layer F.Cu) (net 10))
 (segment (start 137.7625 93.175) (end 139.525 93.175) (width 0.2) (layer B.Cu) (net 11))
 (via (at 140.454 92.5) (size 0.6) (drill 0.4) (layers F.Cu B.Cu) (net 11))
 (segment (start 139.779 93.175) (end 140.454 92.5) (width 0.254) (layer B.Cu) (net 11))
 (segment (start 139.525 93.175) (end 139.779 93.175) (width 0.254) (layer B.Cu) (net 11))
 (via (at 140 88.5) (size 0.6) (drill 0.4) (layers F.Cu B.Cu) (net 11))
 (segment (start 140.454 88.954) (end 140 88.5) (width 0.254) (layer F.Cu) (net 11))
 (segment (start 140.454 92.5) (end 140.454 88.954) (width 0.254) (layer F.Cu) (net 11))
 (segment (start 140.25 88.5) (end 141 87.75) (width 0.254) (layer B.Cu) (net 11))
 (segment (start 140 88.5) (end 140.25 88.5) (width 0.254) (layer B.Cu) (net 11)))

